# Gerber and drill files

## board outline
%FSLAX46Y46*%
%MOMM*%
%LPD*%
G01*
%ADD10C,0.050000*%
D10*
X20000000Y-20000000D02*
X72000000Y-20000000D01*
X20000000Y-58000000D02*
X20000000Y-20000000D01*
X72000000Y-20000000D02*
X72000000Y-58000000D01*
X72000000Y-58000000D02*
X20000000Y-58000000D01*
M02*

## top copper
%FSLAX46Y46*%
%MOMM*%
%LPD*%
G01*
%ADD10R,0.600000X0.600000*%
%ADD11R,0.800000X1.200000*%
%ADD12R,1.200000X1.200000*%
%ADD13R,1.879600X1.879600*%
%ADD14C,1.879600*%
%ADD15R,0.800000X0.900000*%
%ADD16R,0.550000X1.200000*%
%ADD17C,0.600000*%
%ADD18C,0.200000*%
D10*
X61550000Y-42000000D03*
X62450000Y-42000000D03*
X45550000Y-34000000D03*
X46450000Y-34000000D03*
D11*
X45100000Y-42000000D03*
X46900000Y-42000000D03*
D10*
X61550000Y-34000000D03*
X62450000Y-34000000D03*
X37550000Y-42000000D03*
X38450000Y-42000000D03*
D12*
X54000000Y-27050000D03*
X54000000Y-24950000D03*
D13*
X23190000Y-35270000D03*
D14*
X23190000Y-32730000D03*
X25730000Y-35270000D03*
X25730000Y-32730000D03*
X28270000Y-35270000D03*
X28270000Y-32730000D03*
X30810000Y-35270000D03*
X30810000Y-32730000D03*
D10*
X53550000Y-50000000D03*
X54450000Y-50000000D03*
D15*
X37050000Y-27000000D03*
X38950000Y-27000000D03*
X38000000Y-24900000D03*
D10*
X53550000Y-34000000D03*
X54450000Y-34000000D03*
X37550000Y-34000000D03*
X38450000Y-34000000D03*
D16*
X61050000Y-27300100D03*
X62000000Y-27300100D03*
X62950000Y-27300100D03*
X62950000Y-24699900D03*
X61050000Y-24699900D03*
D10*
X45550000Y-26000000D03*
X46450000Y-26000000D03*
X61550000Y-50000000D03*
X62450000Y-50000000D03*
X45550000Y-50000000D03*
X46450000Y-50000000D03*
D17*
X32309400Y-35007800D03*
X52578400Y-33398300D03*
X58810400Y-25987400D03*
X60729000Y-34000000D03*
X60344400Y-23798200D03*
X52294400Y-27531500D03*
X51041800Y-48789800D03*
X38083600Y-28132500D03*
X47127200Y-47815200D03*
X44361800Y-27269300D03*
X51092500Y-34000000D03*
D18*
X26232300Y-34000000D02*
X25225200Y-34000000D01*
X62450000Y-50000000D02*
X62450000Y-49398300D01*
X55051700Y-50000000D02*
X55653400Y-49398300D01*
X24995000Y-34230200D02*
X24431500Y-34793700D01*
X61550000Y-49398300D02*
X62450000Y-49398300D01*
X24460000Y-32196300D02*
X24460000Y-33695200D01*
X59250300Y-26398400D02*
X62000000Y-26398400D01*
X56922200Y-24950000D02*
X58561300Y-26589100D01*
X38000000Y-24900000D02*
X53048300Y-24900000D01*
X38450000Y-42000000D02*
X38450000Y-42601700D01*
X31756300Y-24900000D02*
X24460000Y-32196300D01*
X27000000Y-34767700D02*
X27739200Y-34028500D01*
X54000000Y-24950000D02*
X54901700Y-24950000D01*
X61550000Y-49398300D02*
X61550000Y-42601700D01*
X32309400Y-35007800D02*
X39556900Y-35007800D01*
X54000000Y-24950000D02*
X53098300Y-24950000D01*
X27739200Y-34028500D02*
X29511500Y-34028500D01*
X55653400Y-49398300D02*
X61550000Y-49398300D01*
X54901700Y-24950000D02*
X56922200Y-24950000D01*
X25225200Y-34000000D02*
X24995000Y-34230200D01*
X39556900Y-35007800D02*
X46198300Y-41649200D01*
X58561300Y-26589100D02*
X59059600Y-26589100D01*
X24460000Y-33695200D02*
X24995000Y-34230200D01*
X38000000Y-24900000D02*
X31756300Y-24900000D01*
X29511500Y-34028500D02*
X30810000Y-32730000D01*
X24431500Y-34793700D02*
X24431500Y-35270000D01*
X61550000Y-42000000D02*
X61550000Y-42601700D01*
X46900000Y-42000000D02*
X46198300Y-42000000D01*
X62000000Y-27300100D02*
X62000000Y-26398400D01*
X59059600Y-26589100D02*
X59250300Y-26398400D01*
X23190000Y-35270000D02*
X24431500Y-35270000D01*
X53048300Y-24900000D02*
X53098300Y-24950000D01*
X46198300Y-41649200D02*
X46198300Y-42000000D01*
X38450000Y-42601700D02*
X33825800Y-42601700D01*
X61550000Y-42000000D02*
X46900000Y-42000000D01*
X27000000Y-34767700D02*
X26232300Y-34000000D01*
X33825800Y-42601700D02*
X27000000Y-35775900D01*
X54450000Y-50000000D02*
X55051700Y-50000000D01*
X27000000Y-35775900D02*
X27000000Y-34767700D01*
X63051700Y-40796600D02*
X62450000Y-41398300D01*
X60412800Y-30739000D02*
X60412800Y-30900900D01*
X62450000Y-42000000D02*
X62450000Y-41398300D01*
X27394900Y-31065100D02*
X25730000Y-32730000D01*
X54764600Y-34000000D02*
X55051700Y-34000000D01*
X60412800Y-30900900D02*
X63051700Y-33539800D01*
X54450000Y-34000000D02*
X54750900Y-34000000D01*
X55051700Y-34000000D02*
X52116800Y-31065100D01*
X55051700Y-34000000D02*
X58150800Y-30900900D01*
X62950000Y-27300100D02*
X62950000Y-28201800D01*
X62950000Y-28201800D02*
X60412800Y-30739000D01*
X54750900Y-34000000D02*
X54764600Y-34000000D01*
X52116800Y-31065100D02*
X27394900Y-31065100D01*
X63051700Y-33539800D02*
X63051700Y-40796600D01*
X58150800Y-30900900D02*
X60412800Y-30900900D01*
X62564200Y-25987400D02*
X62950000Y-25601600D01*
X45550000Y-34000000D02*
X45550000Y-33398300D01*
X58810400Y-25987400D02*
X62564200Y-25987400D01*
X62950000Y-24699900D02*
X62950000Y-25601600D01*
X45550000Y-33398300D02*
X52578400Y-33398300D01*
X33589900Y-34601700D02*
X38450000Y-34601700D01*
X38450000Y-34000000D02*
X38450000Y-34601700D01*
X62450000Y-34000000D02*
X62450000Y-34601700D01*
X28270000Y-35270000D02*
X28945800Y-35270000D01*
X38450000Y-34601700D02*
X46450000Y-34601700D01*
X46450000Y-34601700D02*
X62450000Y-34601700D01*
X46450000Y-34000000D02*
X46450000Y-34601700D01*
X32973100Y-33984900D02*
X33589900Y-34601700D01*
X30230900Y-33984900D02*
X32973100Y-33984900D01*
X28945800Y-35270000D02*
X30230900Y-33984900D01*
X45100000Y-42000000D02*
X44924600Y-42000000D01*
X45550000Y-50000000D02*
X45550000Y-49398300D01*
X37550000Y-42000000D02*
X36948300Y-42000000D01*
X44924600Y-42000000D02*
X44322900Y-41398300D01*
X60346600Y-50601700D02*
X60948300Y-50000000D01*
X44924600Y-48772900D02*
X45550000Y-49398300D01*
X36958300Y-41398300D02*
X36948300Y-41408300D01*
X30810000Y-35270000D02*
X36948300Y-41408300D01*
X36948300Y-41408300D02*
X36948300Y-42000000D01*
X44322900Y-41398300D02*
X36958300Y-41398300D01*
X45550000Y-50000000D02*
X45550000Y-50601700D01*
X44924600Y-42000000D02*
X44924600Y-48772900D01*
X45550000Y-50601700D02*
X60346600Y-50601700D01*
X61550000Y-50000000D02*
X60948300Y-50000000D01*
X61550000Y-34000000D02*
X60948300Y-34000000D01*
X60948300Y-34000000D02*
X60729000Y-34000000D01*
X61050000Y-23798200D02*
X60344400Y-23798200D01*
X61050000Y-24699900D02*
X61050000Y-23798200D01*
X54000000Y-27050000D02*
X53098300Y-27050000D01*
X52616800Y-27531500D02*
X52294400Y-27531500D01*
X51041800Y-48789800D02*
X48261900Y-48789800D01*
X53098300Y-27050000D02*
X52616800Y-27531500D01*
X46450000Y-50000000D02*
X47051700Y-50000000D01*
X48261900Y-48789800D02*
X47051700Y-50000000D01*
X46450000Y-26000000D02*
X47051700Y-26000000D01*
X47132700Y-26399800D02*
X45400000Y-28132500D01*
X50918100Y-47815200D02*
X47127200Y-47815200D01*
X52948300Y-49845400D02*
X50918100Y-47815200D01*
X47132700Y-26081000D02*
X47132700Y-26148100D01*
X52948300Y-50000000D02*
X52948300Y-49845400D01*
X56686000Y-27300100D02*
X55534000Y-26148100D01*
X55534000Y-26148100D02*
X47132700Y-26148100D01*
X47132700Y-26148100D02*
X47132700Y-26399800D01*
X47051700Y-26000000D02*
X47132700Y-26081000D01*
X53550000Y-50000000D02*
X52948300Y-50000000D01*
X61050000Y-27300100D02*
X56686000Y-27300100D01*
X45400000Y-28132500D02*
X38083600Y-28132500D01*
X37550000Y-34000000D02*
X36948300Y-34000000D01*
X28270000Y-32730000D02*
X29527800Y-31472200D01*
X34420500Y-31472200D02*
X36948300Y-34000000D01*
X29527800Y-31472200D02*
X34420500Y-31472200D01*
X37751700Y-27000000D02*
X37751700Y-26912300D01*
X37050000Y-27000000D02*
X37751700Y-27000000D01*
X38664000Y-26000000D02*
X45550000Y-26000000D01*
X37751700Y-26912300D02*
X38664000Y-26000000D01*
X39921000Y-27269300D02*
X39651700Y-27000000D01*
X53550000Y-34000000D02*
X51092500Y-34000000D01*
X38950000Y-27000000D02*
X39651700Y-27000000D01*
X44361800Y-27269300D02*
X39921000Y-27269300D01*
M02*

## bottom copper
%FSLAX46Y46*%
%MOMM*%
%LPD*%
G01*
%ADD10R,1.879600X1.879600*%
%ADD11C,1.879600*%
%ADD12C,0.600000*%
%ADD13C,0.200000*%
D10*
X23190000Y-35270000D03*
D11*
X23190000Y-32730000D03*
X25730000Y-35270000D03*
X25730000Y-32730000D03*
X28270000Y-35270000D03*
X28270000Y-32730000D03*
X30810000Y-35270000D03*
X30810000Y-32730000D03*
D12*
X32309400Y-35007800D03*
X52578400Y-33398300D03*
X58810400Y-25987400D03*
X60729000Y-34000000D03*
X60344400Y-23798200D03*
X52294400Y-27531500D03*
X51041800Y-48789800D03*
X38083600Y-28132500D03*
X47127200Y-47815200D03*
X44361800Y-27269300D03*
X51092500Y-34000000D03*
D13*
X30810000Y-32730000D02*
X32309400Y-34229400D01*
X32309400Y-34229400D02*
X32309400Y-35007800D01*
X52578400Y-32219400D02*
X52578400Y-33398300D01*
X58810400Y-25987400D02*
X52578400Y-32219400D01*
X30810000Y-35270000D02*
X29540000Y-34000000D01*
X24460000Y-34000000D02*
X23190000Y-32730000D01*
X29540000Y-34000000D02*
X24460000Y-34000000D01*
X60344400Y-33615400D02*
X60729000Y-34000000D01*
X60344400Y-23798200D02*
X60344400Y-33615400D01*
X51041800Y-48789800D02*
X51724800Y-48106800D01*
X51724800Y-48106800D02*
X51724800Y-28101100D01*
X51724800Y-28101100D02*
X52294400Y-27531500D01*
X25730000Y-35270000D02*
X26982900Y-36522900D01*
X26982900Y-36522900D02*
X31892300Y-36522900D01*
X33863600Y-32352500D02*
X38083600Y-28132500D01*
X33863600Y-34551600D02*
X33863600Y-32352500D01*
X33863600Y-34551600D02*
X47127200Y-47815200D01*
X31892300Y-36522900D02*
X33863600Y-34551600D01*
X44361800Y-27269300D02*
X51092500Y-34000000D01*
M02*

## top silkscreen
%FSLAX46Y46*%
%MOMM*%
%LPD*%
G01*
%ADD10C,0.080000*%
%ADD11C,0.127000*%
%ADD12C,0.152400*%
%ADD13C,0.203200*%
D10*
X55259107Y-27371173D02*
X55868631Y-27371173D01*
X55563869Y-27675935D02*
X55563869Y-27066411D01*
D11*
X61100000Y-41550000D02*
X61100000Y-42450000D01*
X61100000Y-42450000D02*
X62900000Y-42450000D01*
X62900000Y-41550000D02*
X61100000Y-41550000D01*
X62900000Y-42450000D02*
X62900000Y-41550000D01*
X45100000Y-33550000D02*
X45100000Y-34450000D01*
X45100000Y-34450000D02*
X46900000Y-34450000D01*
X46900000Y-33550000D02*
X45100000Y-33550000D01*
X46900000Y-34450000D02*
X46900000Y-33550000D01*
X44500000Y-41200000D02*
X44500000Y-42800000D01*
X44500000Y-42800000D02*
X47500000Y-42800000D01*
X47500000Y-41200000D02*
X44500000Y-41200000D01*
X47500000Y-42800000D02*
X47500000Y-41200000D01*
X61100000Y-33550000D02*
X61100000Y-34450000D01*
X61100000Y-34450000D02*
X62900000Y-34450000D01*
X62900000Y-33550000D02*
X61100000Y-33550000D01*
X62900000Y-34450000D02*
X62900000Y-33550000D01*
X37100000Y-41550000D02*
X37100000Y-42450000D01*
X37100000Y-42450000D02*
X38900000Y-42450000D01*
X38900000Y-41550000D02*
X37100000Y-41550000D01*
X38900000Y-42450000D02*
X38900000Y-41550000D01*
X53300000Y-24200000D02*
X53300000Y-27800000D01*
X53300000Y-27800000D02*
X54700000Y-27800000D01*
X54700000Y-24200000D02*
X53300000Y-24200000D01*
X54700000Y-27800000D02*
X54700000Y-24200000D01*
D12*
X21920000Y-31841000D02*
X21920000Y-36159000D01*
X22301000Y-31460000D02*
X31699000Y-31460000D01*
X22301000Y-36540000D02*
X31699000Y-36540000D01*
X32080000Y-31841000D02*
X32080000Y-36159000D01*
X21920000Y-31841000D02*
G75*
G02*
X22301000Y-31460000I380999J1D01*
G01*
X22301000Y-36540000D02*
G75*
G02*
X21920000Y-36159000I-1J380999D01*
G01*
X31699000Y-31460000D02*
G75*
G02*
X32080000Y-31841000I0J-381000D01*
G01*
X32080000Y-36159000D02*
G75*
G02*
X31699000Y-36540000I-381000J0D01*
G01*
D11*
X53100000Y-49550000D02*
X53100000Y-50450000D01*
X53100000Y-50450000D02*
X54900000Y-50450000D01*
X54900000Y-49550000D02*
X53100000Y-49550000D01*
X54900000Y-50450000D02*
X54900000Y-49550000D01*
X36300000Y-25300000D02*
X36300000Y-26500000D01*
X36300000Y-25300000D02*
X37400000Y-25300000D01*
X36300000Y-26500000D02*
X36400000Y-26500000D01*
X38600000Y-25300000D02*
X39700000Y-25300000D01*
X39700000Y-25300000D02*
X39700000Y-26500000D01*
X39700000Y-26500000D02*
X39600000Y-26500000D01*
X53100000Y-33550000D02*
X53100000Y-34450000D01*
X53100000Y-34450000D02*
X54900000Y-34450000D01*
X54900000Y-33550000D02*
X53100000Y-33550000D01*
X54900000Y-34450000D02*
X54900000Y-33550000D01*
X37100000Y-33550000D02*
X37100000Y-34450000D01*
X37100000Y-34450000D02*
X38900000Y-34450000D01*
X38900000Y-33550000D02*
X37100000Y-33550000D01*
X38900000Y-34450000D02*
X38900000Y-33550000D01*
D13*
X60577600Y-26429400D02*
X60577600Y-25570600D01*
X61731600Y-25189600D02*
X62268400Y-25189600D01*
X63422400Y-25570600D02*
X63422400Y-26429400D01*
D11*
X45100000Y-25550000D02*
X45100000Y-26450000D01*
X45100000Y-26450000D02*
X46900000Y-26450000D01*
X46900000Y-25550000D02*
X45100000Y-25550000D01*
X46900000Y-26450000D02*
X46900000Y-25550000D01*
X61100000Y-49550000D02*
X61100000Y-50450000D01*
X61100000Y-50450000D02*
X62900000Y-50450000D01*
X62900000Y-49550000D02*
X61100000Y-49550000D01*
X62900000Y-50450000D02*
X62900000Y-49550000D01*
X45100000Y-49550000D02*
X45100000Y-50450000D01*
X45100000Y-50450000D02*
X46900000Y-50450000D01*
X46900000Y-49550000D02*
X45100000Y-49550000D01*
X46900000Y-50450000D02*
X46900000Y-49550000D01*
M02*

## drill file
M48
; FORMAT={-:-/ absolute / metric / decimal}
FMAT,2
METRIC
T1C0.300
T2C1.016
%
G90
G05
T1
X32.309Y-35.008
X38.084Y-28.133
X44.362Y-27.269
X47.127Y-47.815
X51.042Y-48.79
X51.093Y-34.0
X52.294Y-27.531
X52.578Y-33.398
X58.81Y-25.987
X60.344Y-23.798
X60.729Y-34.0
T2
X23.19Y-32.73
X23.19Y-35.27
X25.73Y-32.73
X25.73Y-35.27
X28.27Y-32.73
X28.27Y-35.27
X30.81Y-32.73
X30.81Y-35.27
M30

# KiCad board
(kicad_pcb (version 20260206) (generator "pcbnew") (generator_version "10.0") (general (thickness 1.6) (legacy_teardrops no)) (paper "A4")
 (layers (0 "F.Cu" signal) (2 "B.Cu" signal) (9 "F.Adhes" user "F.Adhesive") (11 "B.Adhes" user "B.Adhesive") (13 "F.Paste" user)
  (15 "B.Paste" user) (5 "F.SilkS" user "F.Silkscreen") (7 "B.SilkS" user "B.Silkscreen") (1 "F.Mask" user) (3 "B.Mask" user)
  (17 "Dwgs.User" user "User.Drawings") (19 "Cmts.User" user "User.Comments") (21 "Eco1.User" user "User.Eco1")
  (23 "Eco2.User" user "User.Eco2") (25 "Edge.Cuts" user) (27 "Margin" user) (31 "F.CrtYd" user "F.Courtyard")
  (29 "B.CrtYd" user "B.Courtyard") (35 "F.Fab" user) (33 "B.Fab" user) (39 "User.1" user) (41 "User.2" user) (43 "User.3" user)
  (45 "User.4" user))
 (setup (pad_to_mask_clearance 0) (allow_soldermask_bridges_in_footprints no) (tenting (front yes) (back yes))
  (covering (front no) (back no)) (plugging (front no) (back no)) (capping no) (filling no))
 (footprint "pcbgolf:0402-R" (layer "F.Cu") (at 62 42)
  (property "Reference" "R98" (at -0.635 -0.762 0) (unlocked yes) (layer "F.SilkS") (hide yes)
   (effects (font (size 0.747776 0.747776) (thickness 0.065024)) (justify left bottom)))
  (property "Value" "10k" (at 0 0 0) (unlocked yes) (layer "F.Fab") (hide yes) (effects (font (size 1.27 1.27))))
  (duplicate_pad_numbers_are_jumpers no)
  (fp_line (start -0.9 -0.45) (end -0.9 0.45) (stroke (width 0.127) (type solid)) (layer "F.SilkS"))
  (fp_line (start -0.9 0.45) (end 0.9 0.45) (stroke (width 0.127) (type solid)) (layer "F.SilkS"))
  (fp_line (start 0.9 -0.45) (end -0.9 -0.45) (stroke (width 0.127) (type solid)) (layer "F.SilkS"))
  (fp_line (start 0.9 0.45) (end 0.9 -0.45) (stroke (width 0.127) (type solid)) (layer "F.SilkS"))
  (pad "1" smd rect (at -0.45 0) (size 0.6 0.6) (layers "F.Cu" "F.Mask" "F.Paste") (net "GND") (solder_mask_margin 0.0508)
   (solder_paste_margin 0) (thermal_bridge_angle 0))
  (pad "2" smd rect (at 0.45 0) (size 0.6 0.6) (layers "F.Cu" "F.Mask" "F.Paste") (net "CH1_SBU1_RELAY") (solder_mask_margin 0.0508)
   (solder_paste_margin 0) (thermal_bridge_angle 0)))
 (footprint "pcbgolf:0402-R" (layer "F.Cu") (at 46 34)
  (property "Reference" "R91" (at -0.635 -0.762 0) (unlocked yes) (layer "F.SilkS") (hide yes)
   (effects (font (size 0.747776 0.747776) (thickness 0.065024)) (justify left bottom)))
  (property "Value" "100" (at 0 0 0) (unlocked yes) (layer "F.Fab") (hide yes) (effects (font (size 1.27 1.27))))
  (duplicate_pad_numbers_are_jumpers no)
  (fp_line (start -0.9 -0.45) (end -0.9 0.45) (stroke (width 0.127) (type solid)) (layer "F.SilkS"))
  (fp_line (start -0.9 0.45) (end 0.9 0.45) (stroke (width 0.127) (type solid)) (layer "F.SilkS"))
  (fp_line (start 0.9 -0.45) (end -0.9 -0.45) (stroke (width 0.127) (type solid)) (layer "F.SilkS"))
  (fp_line (start 0.9 0.45) (end 0.9 -0.45) (stroke (width 0.127) (type solid)) (layer "F.SilkS"))
  (pad "1" smd rect (at -0.45 0) (size 0.6 0.6) (layers "F.Cu" "F.Mask" "F.Paste") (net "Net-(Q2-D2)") (solder_mask_margin 0.0508)
   (solder_paste_margin 0) (thermal_bridge_angle 0))
  (pad "2" smd rect (at 0.45 0) (size 0.6 0.6) (layers "F.Cu" "F.Mask" "F.Paste") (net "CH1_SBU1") (solder_mask_margin 0.0508)
   (solder_paste_margin 0) (thermal_bridge_angle 0)))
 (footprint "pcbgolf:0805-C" (layer "F.Cu") (at 46 42)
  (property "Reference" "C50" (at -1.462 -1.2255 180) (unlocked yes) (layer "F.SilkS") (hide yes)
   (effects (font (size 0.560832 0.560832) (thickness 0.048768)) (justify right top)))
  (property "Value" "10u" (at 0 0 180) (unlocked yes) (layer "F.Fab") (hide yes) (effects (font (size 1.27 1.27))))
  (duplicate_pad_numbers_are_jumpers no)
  (fp_line (start -1.5 -0.8) (end -1.5 0.8) (stroke (width 0.127) (type solid)) (layer "F.SilkS"))
  (fp_line (start -1.5 0.8) (end 1.5 0.8) (stroke (width 0.127) (type solid)) (layer "F.SilkS"))
  (fp_line (start 1.5 -0.8) (end -1.5 -0.8) (stroke (width 0.127) (type solid)) (layer "F.SilkS"))
  (fp_line (start 1.5 0.8) (end 1.5 -0.8) (stroke (width 0.127) (type solid)) (layer "F.SilkS"))
  (pad "1" smd rect (at -0.9 0) (size 0.8 1.2) (layers "F.Cu" "F.Mask" "F.Paste") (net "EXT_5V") (solder_mask_margin 0.0508)
   (solder_paste_margin 0) (thermal_bridge_angle 0))
  (pad "2" smd rect (at 0.9 0) (size 0.8 1.2) (layers "F.Cu" "F.Mask" "F.Paste") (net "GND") (solder_mask_margin 0.0508)
   (solder_paste_margin 0) (thermal_bridge_angle 0)))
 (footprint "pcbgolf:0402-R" (layer "F.Cu") (at 62 34)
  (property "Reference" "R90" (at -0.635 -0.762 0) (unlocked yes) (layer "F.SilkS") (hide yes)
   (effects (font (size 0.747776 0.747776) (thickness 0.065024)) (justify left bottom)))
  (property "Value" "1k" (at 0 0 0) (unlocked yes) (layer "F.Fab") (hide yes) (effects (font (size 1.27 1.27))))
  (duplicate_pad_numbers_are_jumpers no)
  (fp_line (start -0.9 -0.45) (end -0.9 0.45) (stroke (width 0.127) (type solid)) (layer "F.SilkS"))
  (fp_line (start -0.9 0.45) (end 0.9 0.45) (stroke (width 0.127) (type solid)) (layer "F.SilkS"))
  (fp_line (start 0.9 -0.45) (end -0.9 -0.45) (stroke (width 0.127) (type solid)) (layer "F.SilkS"))
  (fp_line (start 0.9 0.45) (end 0.9 -0.45) (stroke (width 0.127) (type solid)) (layer "F.SilkS"))
  (pad "1" smd rect (at -0.45 0) (size 0.6 0.6) (layers "F.Cu" "F.Mask" "F.Paste") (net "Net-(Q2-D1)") (solder_mask_margin 0.0508)
   (solder_paste_margin 0) (thermal_bridge_angle 0))
  (pad "2" smd rect (at 0.45 0) (size 0.6 0.6) (layers "F.Cu" "F.Mask" "F.Paste") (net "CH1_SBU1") (solder_mask_margin 0.0508)
   (solder_paste_margin 0) (thermal_bridge_angle 0)))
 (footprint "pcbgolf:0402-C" (layer "F.Cu") (at 38 42)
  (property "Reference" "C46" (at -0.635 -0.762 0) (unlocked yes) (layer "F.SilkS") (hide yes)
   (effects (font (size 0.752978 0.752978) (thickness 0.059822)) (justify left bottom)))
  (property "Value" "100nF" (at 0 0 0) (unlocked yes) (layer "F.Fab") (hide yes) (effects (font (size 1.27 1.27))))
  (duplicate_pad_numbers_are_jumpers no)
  (fp_line (start -0.9 -0.45) (end -0.9 0.45) (stroke (width 0.127) (type solid)) (layer "F.SilkS"))
  (fp_line (start -0.9 0.45) (end 0.9 0.45) (stroke (width 0.127) (type solid)) (layer "F.SilkS"))
  (fp_line (start 0.9 -0.45) (end -0.9 -0.45) (stroke (width 0.127) (type solid)) (layer "F.SilkS"))
  (fp_line (start 0.9 0.45) (end 0.9 -0.45) (stroke (width 0.127) (type solid)) (layer "F.SilkS"))
  (pad "1" smd rect (at -0.45 0) (size 0.6 0.6) (layers "F.Cu" "F.Mask" "F.Paste") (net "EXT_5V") (solder_mask_margin 0.0508)
   (solder_paste_margin 0) (thermal_bridge_angle 0))
  (pad "2" smd rect (at 0.45 0) (size 0.6 0.6) (layers "F.Cu" "F.Mask" "F.Paste") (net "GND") (solder_mask_margin 0.0508)
   (solder_paste_margin 0) (thermal_bridge_angle 0)))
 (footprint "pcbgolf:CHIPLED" (layer "F.Cu") (at 54 26)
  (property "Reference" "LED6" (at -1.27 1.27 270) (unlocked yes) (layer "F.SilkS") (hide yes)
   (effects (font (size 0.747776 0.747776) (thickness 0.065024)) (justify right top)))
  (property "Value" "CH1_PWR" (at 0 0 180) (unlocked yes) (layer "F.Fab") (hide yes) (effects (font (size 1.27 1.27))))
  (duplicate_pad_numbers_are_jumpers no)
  (fp_line (start -0.7 -1.8) (end -0.7 1.8) (stroke (width 0.127) (type solid)) (layer "F.SilkS"))
  (fp_line (start -0.7 1.8) (end 0.7 1.8) (stroke (width 0.127) (type solid)) (layer "F.SilkS"))
  (fp_line (start 0.7 -1.8) (end -0.7 -1.8) (stroke (width 0.127) (type solid)) (layer "F.SilkS"))
  (fp_line (start 0.7 1.8) (end 0.7 -1.8) (stroke (width 0.127) (type solid)) (layer "F.SilkS"))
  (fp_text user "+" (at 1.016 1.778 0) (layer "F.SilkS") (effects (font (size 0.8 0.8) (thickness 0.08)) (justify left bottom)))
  (pad "A" smd rect (at 0 1.05) (size 1.2 1.2) (layers "F.Cu" "F.Mask" "F.Paste") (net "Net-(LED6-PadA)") (solder_mask_margin 0.0508)
   (solder_paste_margin 0) (thermal_bridge_angle 0))
  (pad "C" smd rect (at 0 -1.05) (size 1.2 1.2) (layers "F.Cu" "F.Mask" "F.Paste") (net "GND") (solder_mask_margin 0.0508)
   (solder_paste_margin 0) (thermal_bridge_angle 0)))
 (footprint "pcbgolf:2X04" (layer "F.Cu") (at 27 34)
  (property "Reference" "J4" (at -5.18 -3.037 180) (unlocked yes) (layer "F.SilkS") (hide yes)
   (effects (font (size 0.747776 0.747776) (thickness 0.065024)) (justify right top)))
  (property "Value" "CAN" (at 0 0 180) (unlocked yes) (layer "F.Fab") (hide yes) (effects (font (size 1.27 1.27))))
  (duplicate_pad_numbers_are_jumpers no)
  (fp_line (start -5.08 -2.159) (end -5.08 2.159) (stroke (width 0.1524) (type solid)) (layer "F.SilkS"))
  (fp_line (start -4.699 -2.54) (end 4.699 -2.54) (stroke (width 0.1524) (type solid)) (layer "F.SilkS"))
  (fp_line (start -4.699 2.54) (end 4.699 2.54) (stroke (width 0.1524) (type solid)) (layer "F.SilkS"))
  (fp_line (start 5.08 -2.159) (end 5.08 2.159) (stroke (width 0.1524) (type solid)) (layer "F.SilkS"))
  (fp_arc (start -5.08 -2.159) (mid -4.968408 -2.428408) (end -4.699 -2.54) (stroke (width 0.1524) (type solid)) (layer "F.SilkS"))
  (fp_arc (start -4.699 2.54) (mid -4.968408 2.428408) (end -5.08 2.159) (stroke (width 0.1524) (type solid)) (layer "F.SilkS"))
  (fp_arc (start 4.699 -2.54) (mid 4.968408 -2.428408) (end 5.08 -2.159) (stroke (width 0.1524) (type solid)) (layer "F.SilkS"))
  (fp_arc (start 5.08 2.159) (mid 4.968408 2.428408) (end 4.699 2.54) (stroke (width 0.1524) (type solid)) (layer "F.SilkS"))
  (pad "1" thru_hole rect (at -3.81 1.27 90) (size 1.8796 1.8796) (drill 1.016) (layers "*.Cu" "*.Mask") (remove_unused_layers no)
   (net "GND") (solder_mask_margin 0.0508) (thermal_bridge_angle 0))
  (pad "2" thru_hole circle (at -3.81 -1.27 90) (size 1.8796 1.8796) (drill 1.016) (layers "*.Cu" "*.Mask") (remove_unused_layers no)
   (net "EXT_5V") (solder_mask_margin 0.0508) (thermal_bridge_angle 0))
  (pad "3" thru_hole circle (at -1.27 1.27 90) (size 1.8796 1.8796) (drill 1.016) (layers "*.Cu" "*.Mask") (remove_unused_layers no)
   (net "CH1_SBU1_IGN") (solder_mask_margin 0.0508) (thermal_bridge_angle 0))
  (pad "4" thru_hole circle (at -1.27 -1.27 90) (size 1.8796 1.8796) (drill 1.016) (layers "*.Cu" "*.Mask") (remove_unused_layers no)
   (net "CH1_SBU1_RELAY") (solder_mask_margin 0.0508) (thermal_bridge_angle 0))
  (pad "5" thru_hole circle (at 1.27 1.27 90) (size 1.8796 1.8796) (drill 1.016) (layers "*.Cu" "*.Mask") (remove_unused_layers no)
   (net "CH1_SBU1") (solder_mask_margin 0.0508) (thermal_bridge_angle 0))
  (pad "6" thru_hole circle (at 1.27 -1.27 90) (size 1.8796 1.8796) (drill 1.016) (layers "*.Cu" "*.Mask") (remove_unused_layers no)
   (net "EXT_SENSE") (solder_mask_margin 0.0508) (thermal_bridge_angle 0))
  (pad "7" thru_hole circle (at 3.81 1.27 90) (size 1.8796 1.8796) (drill 1.016) (layers "*.Cu" "*.Mask") (remove_unused_layers no)
   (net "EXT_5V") (solder_mask_margin 0.0508) (thermal_bridge_angle 0))
  (pad "8" thru_hole circle (at 3.81 -1.27 90) (size 1.8796 1.8796) (drill 1.016) (layers "*.Cu" "*.Mask") (remove_unused_layers no)
   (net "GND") (solder_mask_margin 0.0508) (thermal_bridge_angle 0)))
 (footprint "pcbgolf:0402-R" (layer "F.Cu") (at 54 50)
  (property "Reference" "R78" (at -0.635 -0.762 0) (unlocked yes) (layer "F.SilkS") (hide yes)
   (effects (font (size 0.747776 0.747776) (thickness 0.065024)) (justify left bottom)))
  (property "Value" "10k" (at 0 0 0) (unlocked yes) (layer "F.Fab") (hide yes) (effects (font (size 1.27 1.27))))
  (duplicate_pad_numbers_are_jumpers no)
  (fp_line (start -0.9 -0.45) (end -0.9 0.45) (stroke (width 0.127) (type solid)) (layer "F.SilkS"))
  (fp_line (start -0.9 0.45) (end 0.9 0.45) (stroke (width 0.127) (type solid)) (layer "F.SilkS"))
  (fp_line (start 0.9 -0.45) (end -0.9 -0.45) (stroke (width 0.127) (type solid)) (layer "F.SilkS"))
  (fp_line (start 0.9 0.45) (end 0.9 -0.45) (stroke (width 0.127) (type solid)) (layer "F.SilkS"))
  (pad "1" smd rect (at -0.45 0) (size 0.6 0.6) (layers "F.Cu" "F.Mask" "F.Paste") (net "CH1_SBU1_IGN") (solder_mask_margin 0.0508)
   (solder_paste_margin 0) (thermal_bridge_angle 0))
  (pad "2" smd rect (at 0.45 0) (size 0.6 0.6) (layers "F.Cu" "F.Mask" "F.Paste") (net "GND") (solder_mask_margin 0.0508)
   (solder_paste_margin 0) (thermal_bridge_angle 0)))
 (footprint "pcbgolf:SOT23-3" (layer "F.Cu") (at 38 26)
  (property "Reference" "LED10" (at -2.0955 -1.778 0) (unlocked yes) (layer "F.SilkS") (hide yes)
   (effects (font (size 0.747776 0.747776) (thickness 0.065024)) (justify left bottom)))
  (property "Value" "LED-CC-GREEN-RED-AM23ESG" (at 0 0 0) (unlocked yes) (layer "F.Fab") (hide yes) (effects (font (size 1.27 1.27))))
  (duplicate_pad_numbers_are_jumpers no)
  (fp_line (start -1.7 -0.7) (end -1.7 0.5) (stroke (width 0.127) (type solid)) (layer "F.SilkS"))
  (fp_line (start -1.7 -0.7) (end -0.6 -0.7) (stroke (width 0.127) (type solid)) (layer "F.SilkS"))
  (fp_line (start -1.7 0.5) (end -1.6 0.5) (stroke (width 0.127) (type solid)) (layer "F.SilkS"))
  (fp_line (start 0.6 -0.7) (end 1.7 -0.7) (stroke (width 0.127) (type solid)) (layer "F.SilkS"))
  (fp_line (start 1.7 -0.7) (end 1.7 0.5) (stroke (width 0.127) (type solid)) (layer "F.SilkS"))
  (fp_line (start 1.7 0.5) (end 1.6 0.5) (stroke (width 0.127) (type solid)) (layer "F.SilkS"))
  (pad "1" smd rect (at -0.95 1) (size 0.8 0.9) (layers "F.Cu" "F.Mask" "F.Paste") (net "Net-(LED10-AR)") (solder_mask_margin 0.0508)
   (solder_paste_margin 0) (thermal_bridge_angle 0))
  (pad "2" smd rect (at 0.95 1) (size 0.8 0.9) (layers "F.Cu" "F.Mask" "F.Paste") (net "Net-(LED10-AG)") (solder_mask_margin 0.0508)
   (solder_paste_margin 0) (thermal_bridge_angle 0))
  (pad "3" smd rect (at 0 -1.1) (size 0.8 0.9) (layers "F.Cu" "F.Mask" "F.Paste") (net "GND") (solder_mask_margin 0.0508)
   (solder_paste_margin 0) (thermal_bridge_angle 0)))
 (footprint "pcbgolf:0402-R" (layer "F.Cu") (at 54 34)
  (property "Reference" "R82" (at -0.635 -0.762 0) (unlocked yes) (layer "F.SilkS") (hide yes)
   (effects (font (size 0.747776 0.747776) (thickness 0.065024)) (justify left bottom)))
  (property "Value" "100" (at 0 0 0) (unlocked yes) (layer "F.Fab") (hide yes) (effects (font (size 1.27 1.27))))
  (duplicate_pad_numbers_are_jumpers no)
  (fp_line (start -0.9 -0.45) (end -0.9 0.45) (stroke (width 0.127) (type solid)) (layer "F.SilkS"))
  (fp_line (start -0.9 0.45) (end 0.9 0.45) (stroke (width 0.127) (type solid)) (layer "F.SilkS"))
  (fp_line (start 0.9 -0.45) (end -0.9 -0.45) (stroke (width 0.127) (type solid)) (layer "F.SilkS"))
  (fp_line (start 0.9 0.45) (end 0.9 -0.45) (stroke (width 0.127) (type solid)) (layer "F.SilkS"))
  (pad "1" smd rect (at -0.45 0) (size 0.6 0.6) (layers "F.Cu" "F.Mask" "F.Paste") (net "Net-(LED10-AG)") (solder_mask_margin 0.0508)
   (solder_paste_margin 0) (thermal_bridge_angle 0))
  (pad "2" smd rect (at 0.45 0) (size 0.6 0.6) (layers "F.Cu" "F.Mask" "F.Paste") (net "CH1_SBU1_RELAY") (solder_mask_margin 0.0508)
   (solder_paste_margin 0) (thermal_bridge_angle 0)))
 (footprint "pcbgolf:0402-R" (layer "F.Cu") (at 38 34)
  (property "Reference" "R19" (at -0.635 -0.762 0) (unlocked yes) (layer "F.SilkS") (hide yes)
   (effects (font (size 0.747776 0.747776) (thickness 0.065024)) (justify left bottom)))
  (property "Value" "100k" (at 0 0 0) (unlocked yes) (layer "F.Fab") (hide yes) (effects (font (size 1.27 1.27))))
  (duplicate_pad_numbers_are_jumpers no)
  (fp_line (start -0.9 -0.45) (end -0.9 0.45) (stroke (width 0.127) (type solid)) (layer "F.SilkS"))
  (fp_line (start -0.9 0.45) (end 0.9 0.45) (stroke (width 0.127) (type solid)) (layer "F.SilkS"))
  (fp_line (start 0.9 -0.45) (end -0.9 -0.45) (stroke (width 0.127) (type solid)) (layer "F.SilkS"))
  (fp_line (start 0.9 0.45) (end 0.9 -0.45) (stroke (width 0.127) (type solid)) (layer "F.SilkS"))
  (pad "1" smd rect (at -0.45 0) (size 0.6 0.6) (layers "F.Cu" "F.Mask" "F.Paste") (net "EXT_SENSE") (solder_mask_margin 0.0508)
   (solder_paste_margin 0) (thermal_bridge_angle 0))
  (pad "2" smd rect (at 0.45 0) (size 0.6 0.6) (layers "F.Cu" "F.Mask" "F.Paste") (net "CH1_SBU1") (solder_mask_margin 0.0508)
   (solder_paste_margin 0) (thermal_bridge_angle 0)))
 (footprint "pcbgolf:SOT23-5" (layer "F.Cu") (at 62 26)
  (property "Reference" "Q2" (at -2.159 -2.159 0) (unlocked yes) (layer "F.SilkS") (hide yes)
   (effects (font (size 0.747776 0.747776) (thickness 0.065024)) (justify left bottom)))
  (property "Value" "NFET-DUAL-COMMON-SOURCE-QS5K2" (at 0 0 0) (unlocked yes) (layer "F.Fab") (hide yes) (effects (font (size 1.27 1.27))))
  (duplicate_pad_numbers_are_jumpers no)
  (fp_line (start -1.4224 0.4294) (end -1.4224 -0.4294) (stroke (width 0.2032) (type solid)) (layer "F.SilkS"))
  (fp_line (start -0.2684 -0.8104) (end 0.2684 -0.8104) (stroke (width 0.2032) (type solid)) (layer "F.SilkS"))
  (fp_line (start 1.4224 -0.4294) (end 1.4224 0.4294) (stroke (width 0.2032) (type solid)) (layer "F.SilkS"))
  (pad "1" smd rect (at -0.95 1.3001) (size 0.55 1.2) (layers "F.Cu" "F.Mask" "F.Paste") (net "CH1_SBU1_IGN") (solder_mask_margin 0.0508)
   (solder_paste_margin 0) (thermal_bridge_angle 0))
  (pad "2" smd rect (at 0 1.3001) (size 0.55 1.2) (layers "F.Cu" "F.Mask" "F.Paste") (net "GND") (solder_mask_margin 0.0508)
   (solder_paste_margin 0) (thermal_bridge_angle 0))
  (pad "3" smd rect (at 0.95 1.3001) (size 0.55 1.2) (layers "F.Cu" "F.Mask" "F.Paste") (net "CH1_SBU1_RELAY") (solder_mask_margin 0.0508)
   (solder_paste_margin 0) (thermal_bridge_angle 0))
  (pad "4" smd rect (at 0.95 -1.3001) (size 0.55 1.2) (layers "F.Cu" "F.Mask" "F.Paste") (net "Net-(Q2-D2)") (solder_mask_margin 0.0508)
   (solder_paste_margin 0) (thermal_bridge_angle 0))
  (pad "5" smd rect (at -0.95 -1.3001) (size 0.55 1.2) (layers "F.Cu" "F.Mask" "F.Paste") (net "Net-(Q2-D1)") (solder_mask_margin 0.0508)
   (solder_paste_margin 0) (thermal_bridge_angle 0)))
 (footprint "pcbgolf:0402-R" (layer "F.Cu") (at 46 26)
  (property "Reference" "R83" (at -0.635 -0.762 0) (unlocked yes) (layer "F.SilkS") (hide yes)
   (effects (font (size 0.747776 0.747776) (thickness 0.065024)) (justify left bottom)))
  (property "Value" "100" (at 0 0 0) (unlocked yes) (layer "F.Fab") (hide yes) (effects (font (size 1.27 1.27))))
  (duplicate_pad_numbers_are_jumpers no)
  (fp_line (start -0.9 -0.45) (end -0.9 0.45) (stroke (width 0.127) (type solid)) (layer "F.SilkS"))
  (fp_line (start -0.9 0.45) (end 0.9 0.45) (stroke (width 0.127) (type solid)) (layer "F.SilkS"))
  (fp_line (start 0.9 -0.45) (end -0.9 -0.45) (stroke (width 0.127) (type solid)) (layer "F.SilkS"))
  (fp_line (start 0.9 0.45) (end 0.9 -0.45) (stroke (width 0.127) (type solid)) (layer "F.SilkS"))
  (pad "1" smd rect (at -0.45 0) (size 0.6 0.6) (layers "F.Cu" "F.Mask" "F.Paste") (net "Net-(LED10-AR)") (solder_mask_margin 0.0508)
   (solder_paste_margin 0) (thermal_bridge_angle 0))
  (pad "2" smd rect (at 0.45 0) (size 0.6 0.6) (layers "F.Cu" "F.Mask" "F.Paste") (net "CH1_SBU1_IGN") (solder_mask_margin 0.0508)
   (solder_paste_margin 0) (thermal_bridge_angle 0)))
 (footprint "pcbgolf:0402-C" (layer "F.Cu") (at 62 50)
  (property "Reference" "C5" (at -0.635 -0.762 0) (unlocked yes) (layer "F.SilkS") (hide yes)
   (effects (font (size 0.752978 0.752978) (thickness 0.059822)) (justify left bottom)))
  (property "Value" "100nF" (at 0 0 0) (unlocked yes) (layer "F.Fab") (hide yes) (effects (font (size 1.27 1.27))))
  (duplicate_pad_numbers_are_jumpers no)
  (fp_line (start -0.9 -0.45) (end -0.9 0.45) (stroke (width 0.127) (type solid)) (layer "F.SilkS"))
  (fp_line (start -0.9 0.45) (end 0.9 0.45) (stroke (width 0.127) (type solid)) (layer "F.SilkS"))
  (fp_line (start 0.9 -0.45) (end -0.9 -0.45) (stroke (width 0.127) (type solid)) (layer "F.SilkS"))
  (fp_line (start 0.9 0.45) (end 0.9 -0.45) (stroke (width 0.127) (type solid)) (layer "F.SilkS"))
  (pad "1" smd rect (at -0.45 0) (size 0.6 0.6) (layers "F.Cu" "F.Mask" "F.Paste") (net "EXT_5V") (solder_mask_margin 0.0508)
   (solder_paste_margin 0) (thermal_bridge_angle 0))
  (pad "2" smd rect (at 0.45 0) (size 0.6 0.6) (layers "F.Cu" "F.Mask" "F.Paste") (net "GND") (solder_mask_margin 0.0508)
   (solder_paste_margin 0) (thermal_bridge_angle 0)))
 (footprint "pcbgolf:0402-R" (layer "F.Cu") (at 46 50)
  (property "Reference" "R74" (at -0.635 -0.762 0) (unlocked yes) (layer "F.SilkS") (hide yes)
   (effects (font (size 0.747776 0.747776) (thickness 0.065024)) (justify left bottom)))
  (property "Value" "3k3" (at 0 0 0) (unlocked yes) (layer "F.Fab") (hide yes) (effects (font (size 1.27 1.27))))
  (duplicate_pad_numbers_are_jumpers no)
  (fp_line (start -0.9 -0.45) (end -0.9 0.45) (stroke (width 0.127) (type solid)) (layer "F.SilkS"))
  (fp_line (start -0.9 0.45) (end 0.9 0.45) (stroke (width 0.127) (type solid)) (layer "F.SilkS"))
  (fp_line (start 0.9 -0.45) (end -0.9 -0.45) (stroke (width 0.127) (type solid)) (layer "F.SilkS"))
  (fp_line (start 0.9 0.45) (end 0.9 -0.45) (stroke (width 0.127) (type solid)) (layer "F.SilkS"))
  (pad "1" smd rect (at -0.45 0) (size 0.6 0.6) (layers "F.Cu" "F.Mask" "F.Paste") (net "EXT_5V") (solder_mask_margin 0.0508)
   (solder_paste_margin 0) (thermal_bridge_angle 0))
  (pad "2" smd rect (at 0.45 0) (size 0.6 0.6) (layers "F.Cu" "F.Mask" "F.Paste") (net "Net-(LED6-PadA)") (solder_mask_margin 0.0508)
   (solder_paste_margin 0) (thermal_bridge_angle 0)))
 (gr_line (start 20 20) (end 72 20) (stroke (width 0.05) (type default)) (layer "Edge.Cuts"))
 (gr_line (start 20 58) (end 20 20) (stroke (width 0.05) (type default)) (layer "Edge.Cuts"))
 (gr_line (start 72 20) (end 72 58) (stroke (width 0.05) (type default)) (layer "Edge.Cuts"))
 (gr_line (start 72 58) (end 20 58) (stroke (width 0.05) (type default)) (layer "Edge.Cuts"))
 (segment (start 26.2323 34) (end 25.2252 34) (width 0.2) (layer "F.Cu") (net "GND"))
 (segment (start 62.45 50) (end 62.45 49.3983) (width 0.2) (layer "F.Cu") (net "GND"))
 (segment (start 55.0517 50) (end 55.6534 49.3983) (width 0.2) (layer "F.Cu") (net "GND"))
 (segment (start 24.995 34.2302) (end 24.4315 34.7937) (width 0.2) (layer "F.Cu") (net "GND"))
 (segment (start 61.55 49.3983) (end 62.45 49.3983) (width 0.2) (layer "F.Cu") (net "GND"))
 (segment (start 24.46 32.1963) (end 24.46 33.6952) (width 0.2) (layer "F.Cu") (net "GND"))
 (segment (start 59.2503 26.3984) (end 62 26.3984) (width 0.2) (layer "F.Cu") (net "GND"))
 (segment (start 56.9222 24.95) (end 58.5613 26.5891) (width 0.2) (layer "F.Cu") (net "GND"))
 (segment (start 38 24.9) (end 53.0483 24.9) (width 0.2) (layer "F.Cu") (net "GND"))
 (segment (start 38.45 42) (end 38.45 42.6017) (width 0.2) (layer "F.Cu") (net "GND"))
 (segment (start 31.7563 24.9) (end 24.46 32.1963) (width 0.2) (layer "F.Cu") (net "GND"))
 (segment (start 27 34.7677) (end 27.7392 34.0285) (width 0.2) (layer "F.Cu") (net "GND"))
 (segment (start 54 24.95) (end 54.9017 24.95) (width 0.2) (layer "F.Cu") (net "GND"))
 (segment (start 61.55 49.3983) (end 61.55 42.6017) (width 0.2) (layer "F.Cu") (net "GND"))
 (segment (start 32.3094 35.0078) (end 39.5569 35.0078) (width 0.2) (layer "F.Cu") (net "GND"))
 (segment (start 54 24.95) (end 53.0983 24.95) (width 0.2) (layer "F.Cu") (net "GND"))
 (segment (start 27.7392 34.0285) (end 29.5115 34.0285) (width 0.2) (layer "F.Cu") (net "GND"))
 (segment (start 55.6534 49.3983) (end 61.55 49.3983) (width 0.2) (layer "F.Cu") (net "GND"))
 (segment (start 54.9017 24.95) (end 56.9222 24.95) (width 0.2) (layer "F.Cu") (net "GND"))
 (segment (start 25.2252 34) (end 24.995 34.2302) (width 0.2) (layer "F.Cu") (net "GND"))
 (segment (start 39.5569 35.0078) (end 46.1983 41.6492) (width 0.2) (layer "F.Cu") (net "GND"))
 (segment (start 58.5613 26.5891) (end 59.0596 26.5891) (width 0.2) (layer "F.Cu") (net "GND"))
 (segment (start 24.46 33.6952) (end 24.995 34.2302) (width 0.2) (layer "F.Cu") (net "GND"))
 (segment (start 38 24.9) (end 31.7563 24.9) (width 0.2) (layer "F.Cu") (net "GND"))
 (segment (start 29.5115 34.0285) (end 30.81 32.73) (width 0.2) (layer "F.Cu") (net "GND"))
 (segment (start 24.4315 34.7937) (end 24.4315 35.27) (width 0.2) (layer "F.Cu") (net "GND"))
 (segment (start 61.55 42) (end 61.55 42.6017) (width 0.2) (layer "F.Cu") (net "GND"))
 (segment (start 46.9 42) (end 46.1983 42) (width 0.2) (layer "F.Cu") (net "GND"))
 (segment (start 62 27.3001) (end 62 26.3984) (width 0.2) (layer "F.Cu") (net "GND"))
 (segment (start 59.0596 26.5891) (end 59.2503 26.3984) (width 0.2) (layer "F.Cu") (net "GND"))
 (segment (start 23.19 35.27) (end 24.4315 35.27) (width 0.2) (layer "F.Cu") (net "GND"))
 (segment (start 53.0483 24.9) (end 53.0983 24.95) (width 0.2) (layer "F.Cu") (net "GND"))
 (segment (start 46.1983 41.6492) (end 46.1983 42) (width 0.2) (layer "F.Cu") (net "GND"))
 (segment (start 38.45 42.6017) (end 33.8258 42.6017) (width 0.2) (layer "F.Cu") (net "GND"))
 (segment (start 61.55 42) (end 46.9 42) (width 0.2) (layer "F.Cu") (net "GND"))
 (segment (start 27 34.7677) (end 26.2323 34) (width 0.2) (layer "F.Cu") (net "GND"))
 (segment (start 33.8258 42.6017) (end 27 35.7759) (width 0.2) (layer "F.Cu") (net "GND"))
 (segment (start 54.45 50) (end 55.0517 50) (width 0.2) (layer "F.Cu") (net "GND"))
 (segment (start 27 35.7759) (end 27 34.7677) (width 0.2) (layer "F.Cu") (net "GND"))
 (via (at 32.3094 35.0078) (size 0.6) (drill 0.3) (layers "F.Cu" "B.Cu") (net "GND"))
 (segment (start 30.81 32.73) (end 32.3094 34.2294) (width 0.2) (layer "B.Cu") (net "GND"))
 (segment (start 32.3094 34.2294) (end 32.3094 35.0078) (width 0.2) (layer "B.Cu") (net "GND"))
 (segment (start 63.0517 40.7966) (end 62.45 41.3983) (width 0.2) (layer "F.Cu") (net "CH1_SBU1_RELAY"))
 (segment (start 60.4128 30.739) (end 60.4128 30.9009) (width 0.2) (layer "F.Cu") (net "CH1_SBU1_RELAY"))
 (segment (start 62.45 42) (end 62.45 41.3983) (width 0.2) (layer "F.Cu") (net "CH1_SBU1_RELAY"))
 (segment (start 27.3949 31.0651) (end 25.73 32.73) (width 0.2) (layer "F.Cu") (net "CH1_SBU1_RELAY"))
 (segment (start 54.7646 34) (end 55.0517 34) (width 0.2) (layer "F.Cu") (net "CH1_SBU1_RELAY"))
 (segment (start 60.4128 30.9009) (end 63.0517 33.5398) (width 0.2) (layer "F.Cu") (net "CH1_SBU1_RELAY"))
 (segment (start 54.45 34) (end 54.7509 34) (width 0.2) (layer "F.Cu") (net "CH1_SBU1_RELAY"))
 (segment (start 55.0517 34) (end 52.1168 31.0651) (width 0.2) (layer "F.Cu") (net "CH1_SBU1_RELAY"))
 (segment (start 55.0517 34) (end 58.1508 30.9009) (width 0.2) (layer "F.Cu") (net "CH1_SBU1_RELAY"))
 (segment (start 62.95 27.3001) (end 62.95 28.2018) (width 0.2) (layer "F.Cu") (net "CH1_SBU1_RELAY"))
 (segment (start 62.95 28.2018) (end 60.4128 30.739) (width 0.2) (layer "F.Cu") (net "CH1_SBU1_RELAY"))
 (segment (start 54.7509 34) (end 54.7646 34) (width 0.2) (layer "F.Cu") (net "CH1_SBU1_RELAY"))
 (segment (start 52.1168 31.0651) (end 27.3949 31.0651) (width 0.2) (layer "F.Cu") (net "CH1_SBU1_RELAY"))
 (segment (start 63.0517 33.5398) (end 63.0517 40.7966) (width 0.2) (layer "F.Cu") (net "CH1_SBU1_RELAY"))
 (segment (start 58.1508 30.9009) (end 60.4128 30.9009) (width 0.2) (layer "F.Cu") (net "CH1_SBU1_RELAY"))
 (segment (start 62.5642 25.9874) (end 62.95 25.6016) (width 0.2) (layer "F.Cu") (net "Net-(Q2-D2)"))
 (segment (start 45.55 34) (end 45.55 33.3983) (width 0.2) (layer "F.Cu") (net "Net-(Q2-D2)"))
 (segment (start 58.8104 25.9874) (end 62.5642 25.9874) (width 0.2) (layer "F.Cu") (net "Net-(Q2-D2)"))
 (segment (start 62.95 24.6999) (end 62.95 25.6016) (width 0.2) (layer "F.Cu") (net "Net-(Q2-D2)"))
 (segment (start 45.55 33.3983) (end 52.5784 33.3983) (width 0.2) (layer "F.Cu") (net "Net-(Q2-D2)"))
 (via (at 52.5784 33.3983) (size 0.6) (drill 0.3) (layers "F.Cu" "B.Cu") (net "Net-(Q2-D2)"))
 (via (at 58.8104 25.9874) (size 0.6) (drill 0.3) (layers "F.Cu" "B.Cu") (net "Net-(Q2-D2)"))
 (segment (start 52.5784 32.2194) (end 52.5784 33.3983) (width 0.2) (layer "B.Cu") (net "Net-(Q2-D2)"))
 (segment (start 58.8104 25.9874) (end 52.5784 32.2194) (width 0.2) (layer "B.Cu") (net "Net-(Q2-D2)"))
 (segment (start 33.5899 34.6017) (end 38.45 34.6017) (width 0.2) (layer "F.Cu") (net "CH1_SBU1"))
 (segment (start 38.45 34) (end 38.45 34.6017) (width 0.2) (layer "F.Cu") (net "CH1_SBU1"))
 (segment (start 62.45 34) (end 62.45 34.6017) (width 0.2) (layer "F.Cu") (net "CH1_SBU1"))
 (segment (start 28.27 35.27) (end 28.9458 35.27) (width 0.2) (layer "F.Cu") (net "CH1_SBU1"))
 (segment (start 38.45 34.6017) (end 46.45 34.6017) (width 0.2) (layer "F.Cu") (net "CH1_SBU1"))
 (segment (start 46.45 34.6017) (end 62.45 34.6017) (width 0.2) (layer "F.Cu") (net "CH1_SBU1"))
 (segment (start 46.45 34) (end 46.45 34.6017) (width 0.2) (layer "F.Cu") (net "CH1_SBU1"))
 (segment (start 32.9731 33.9849) (end 33.5899 34.6017) (width 0.2) (layer "F.Cu") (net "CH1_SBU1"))
 (segment (start 30.2309 33.9849) (end 32.9731 33.9849) (width 0.2) (layer "F.Cu") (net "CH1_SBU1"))
 (segment (start 28.9458 35.27) (end 30.2309 33.9849) (width 0.2) (layer "F.Cu") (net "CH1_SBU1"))
 (segment (start 45.1 42) (end 44.9246 42) (width 0.2) (layer "F.Cu") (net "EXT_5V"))
 (segment (start 45.55 50) (end 45.55 49.3983) (width 0.2) (layer "F.Cu") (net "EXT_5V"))
 (segment (start 37.55 42) (end 36.9483 42) (width 0.2) (layer "F.Cu") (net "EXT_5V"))
 (segment (start 44.9246 42) (end 44.3229 41.3983) (width 0.2) (layer "F.Cu") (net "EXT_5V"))
 (segment (start 60.3466 50.6017) (end 60.9483 50) (width 0.2) (layer "F.Cu") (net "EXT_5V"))
 (segment (start 44.9246 48.7729) (end 45.55 49.3983) (width 0.2) (layer "F.Cu") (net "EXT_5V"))
 (segment (start 36.9583 41.3983) (end 36.9483 41.4083) (width 0.2) (layer "F.Cu") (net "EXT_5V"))
 (segment (start 30.81 35.27) (end 36.9483 41.4083) (width 0.2) (layer "F.Cu") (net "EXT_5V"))
 (segment (start 36.9483 41.4083) (end 36.9483 42) (width 0.2) (layer "F.Cu") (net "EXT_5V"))
 (segment (start 44.3229 41.3983) (end 36.9583 41.3983) (width 0.2) (layer "F.Cu") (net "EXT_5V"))
 (segment (start 45.55 50) (end 45.55 50.6017) (width 0.2) (layer "F.Cu") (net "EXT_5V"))
 (segment (start 44.9246 42) (end 44.9246 48.7729) (width 0.2) (layer "F.Cu") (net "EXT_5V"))
 (segment (start 45.55 50.6017) (end 60.3466 50.6017) (width 0.2) (layer "F.Cu") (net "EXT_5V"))
 (segment (start 61.55 50) (end 60.9483 50) (width 0.2) (layer "F.Cu") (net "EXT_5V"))
 (segment (start 30.81 35.27) (end 29.54 34) (width 0.2) (layer "B.Cu") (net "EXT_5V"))
 (segment (start 24.46 34) (end 23.19 32.73) (width 0.2) (layer "B.Cu") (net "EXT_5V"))
 (segment (start 29.54 34) (end 24.46 34) (width 0.2) (layer "B.Cu") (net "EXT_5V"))
 (segment (start 61.55 34) (end 60.9483 34) (width 0.2) (layer "F.Cu") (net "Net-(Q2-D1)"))
 (segment (start 60.9483 34) (end 60.729 34) (width 0.2) (layer "F.Cu") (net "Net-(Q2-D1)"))
 (segment (start 61.05 23.7982) (end 60.3444 23.7982) (width 0.2) (layer "F.Cu") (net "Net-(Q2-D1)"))
 (segment (start 61.05 24.6999) (end 61.05 23.7982) (width 0.2) (layer "F.Cu") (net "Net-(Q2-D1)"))
 (via (at 60.729 34) (size 0.6) (drill 0.3) (layers "F.Cu" "B.Cu") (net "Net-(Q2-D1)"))
 (via (at 60.3444 23.7982) (size 0.6) (drill 0.3) (layers "F.Cu" "B.Cu") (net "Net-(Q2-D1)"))
 (segment (start 60.3444 33.6154) (end 60.729 34) (width 0.2) (layer "B.Cu") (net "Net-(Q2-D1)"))
 (segment (start 60.3444 23.7982) (end 60.3444 33.6154) (width 0.2) (layer "B.Cu") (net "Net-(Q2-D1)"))
 (segment (start 54 27.05) (end 53.0983 27.05) (width 0.2) (layer "F.Cu") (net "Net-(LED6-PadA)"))
 (segment (start 52.6168 27.5315) (end 52.2944 27.5315) (width 0.2) (layer "F.Cu") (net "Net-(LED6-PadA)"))
 (segment (start 51.0418 48.7898) (end 48.2619 48.7898) (width 0.2) (layer "F.Cu") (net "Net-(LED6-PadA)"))
 (segment (start 53.0983 27.05) (end 52.6168 27.5315) (width 0.2) (layer "F.Cu") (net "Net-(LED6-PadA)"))
 (segment (start 46.45 50) (end 47.0517 50) (width 0.2) (layer "F.Cu") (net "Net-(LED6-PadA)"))
 (segment (start 48.2619 48.7898) (end 47.0517 50) (width 0.2) (layer "F.Cu") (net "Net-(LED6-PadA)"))
 (via (at 52.2944 27.5315) (size 0.6) (drill 0.3) (layers "F.Cu" "B.Cu") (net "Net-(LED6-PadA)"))
 (via (at 51.0418 48.7898) (size 0.6) (drill 0.3) (layers "F.Cu" "B.Cu") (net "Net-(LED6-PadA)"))
 (segment (start 51.0418 48.7898) (end 51.7248 48.1068) (width 0.2) (layer "B.Cu") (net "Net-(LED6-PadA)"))
 (segment (start 51.7248 48.1068) (end 51.7248 28.1011) (width 0.2) (layer "B.Cu") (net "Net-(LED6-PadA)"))
 (segment (start 51.7248 28.1011) (end 52.2944 27.5315) (width 0.2) (layer "B.Cu") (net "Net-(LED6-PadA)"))
 (segment (start 46.45 26) (end 47.0517 26) (width 0.2) (layer "F.Cu") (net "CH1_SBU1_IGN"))
 (segment (start 47.1327 26.3998) (end 45.4 28.1325) (width 0.2) (layer "F.Cu") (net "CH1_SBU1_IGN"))
 (segment (start 50.9181 47.8152) (end 47.1272 47.8152) (width 0.2) (layer "F.Cu") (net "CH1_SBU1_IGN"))
 (segment (start 52.9483 49.8454) (end 50.9181 47.8152) (width 0.2) (layer "F.Cu") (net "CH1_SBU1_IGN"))
 (segment (start 47.1327 26.081) (end 47.1327 26.1481) (width 0.2) (layer "F.Cu") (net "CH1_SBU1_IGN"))
 (segment (start 52.9483 50) (end 52.9483 49.8454) (width 0.2) (layer "F.Cu") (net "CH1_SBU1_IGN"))
 (segment (start 56.686 27.3001) (end 55.534 26.1481) (width 0.2) (layer "F.Cu") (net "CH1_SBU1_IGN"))
 (segment (start 55.534 26.1481) (end 47.1327 26.1481) (width 0.2) (layer "F.Cu") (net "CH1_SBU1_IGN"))
 (segment (start 47.1327 26.1481) (end 47.1327 26.3998) (width 0.2) (layer "F.Cu") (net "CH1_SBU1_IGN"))
 (segment (start 47.0517 26) (end 47.1327 26.081) (width 0.2) (layer "F.Cu") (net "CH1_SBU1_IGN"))
 (segment (start 53.55 50) (end 52.9483 50) (width 0.2) (layer "F.Cu") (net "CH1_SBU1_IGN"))
 (segment (start 61.05 27.3001) (end 56.686 27.3001) (width 0.2) (layer "F.Cu") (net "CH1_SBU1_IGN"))
 (segment (start 45.4 28.1325) (end 38.0836 28.1325) (width 0.2) (layer "F.Cu") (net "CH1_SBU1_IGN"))
 (via (at 38.0836 28.1325) (size 0.6) (drill 0.3) (layers "F.Cu" "B.Cu") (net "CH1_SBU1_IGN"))
 (via (at 47.1272 47.8152) (size 0.6) (drill 0.3) (layers "F.Cu" "B.Cu") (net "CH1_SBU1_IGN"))
 (segment (start 25.73 35.27) (end 26.9829 36.5229) (width 0.2) (layer "B.Cu") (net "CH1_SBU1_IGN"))
 (segment (start 26.9829 36.5229) (end 31.8923 36.5229) (width 0.2) (layer "B.Cu") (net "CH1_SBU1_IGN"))
 (segment (start 33.8636 32.3525) (end 38.0836 28.1325) (width 0.2) (layer "B.Cu") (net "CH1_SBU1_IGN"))
 (segment (start 33.8636 34.5516) (end 33.8636 32.3525) (width 0.2) (layer "B.Cu") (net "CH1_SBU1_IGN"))
 (segment (start 33.8636 34.5516) (end 47.1272 47.8152) (width 0.2) (layer "B.Cu") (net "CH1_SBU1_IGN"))
 (segment (start 31.8923 36.5229) (end 33.8636 34.5516) (width 0.2) (layer "B.Cu") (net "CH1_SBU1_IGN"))
 (segment (start 37.55 34) (end 36.9483 34) (width 0.2) (layer "F.Cu") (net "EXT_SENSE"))
 (segment (start 28.27 32.73) (end 29.5278 31.4722) (width 0.2) (layer "F.Cu") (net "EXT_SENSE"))
 (segment (start 34.4205 31.4722) (end 36.9483 34) (width 0.2) (layer "F.Cu") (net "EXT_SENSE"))
 (segment (start 29.5278 31.4722) (end 34.4205 31.4722) (width 0.2) (layer "F.Cu") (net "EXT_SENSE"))
 (segment (start 37.7517 27) (end 37.7517 26.9123) (width 0.2) (layer "F.Cu") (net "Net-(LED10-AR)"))
 (segment (start 37.05 27) (end 37.7517 27) (width 0.2) (layer "F.Cu") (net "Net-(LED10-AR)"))
 (segment (start 38.664 26) (end 45.55 26) (width 0.2) (layer "F.Cu") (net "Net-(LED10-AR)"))
 (segment (start 37.7517 26.9123) (end 38.664 26) (width 0.2) (layer "F.Cu") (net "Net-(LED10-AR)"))
 (segment (start 39.921 27.2693) (end 39.6517 27) (width 0.2) (layer "F.Cu") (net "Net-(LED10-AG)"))
 (segment (start 53.55 34) (end 51.0925 34) (width 0.2) (layer "F.Cu") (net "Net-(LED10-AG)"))
 (segment (start 38.95 27) (end 39.6517 27) (width 0.2) (layer "F.Cu") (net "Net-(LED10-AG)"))
 (segment (start 44.3618 27.2693) (end 39.921 27.2693) (width 0.2) (layer "F.Cu") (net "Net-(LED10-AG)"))
 (via (at 44.3618 27.2693) (size 0.6) (drill 0.3) (layers "F.Cu" "B.Cu") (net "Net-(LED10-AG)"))
 (via (at 51.0925 34) (size 0.6) (drill 0.3) (layers "F.Cu" "B.Cu") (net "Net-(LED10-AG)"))
 (segment (start 44.3618 27.2693) (end 51.0925 34) (width 0.2) (layer "B.Cu") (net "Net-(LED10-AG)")))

